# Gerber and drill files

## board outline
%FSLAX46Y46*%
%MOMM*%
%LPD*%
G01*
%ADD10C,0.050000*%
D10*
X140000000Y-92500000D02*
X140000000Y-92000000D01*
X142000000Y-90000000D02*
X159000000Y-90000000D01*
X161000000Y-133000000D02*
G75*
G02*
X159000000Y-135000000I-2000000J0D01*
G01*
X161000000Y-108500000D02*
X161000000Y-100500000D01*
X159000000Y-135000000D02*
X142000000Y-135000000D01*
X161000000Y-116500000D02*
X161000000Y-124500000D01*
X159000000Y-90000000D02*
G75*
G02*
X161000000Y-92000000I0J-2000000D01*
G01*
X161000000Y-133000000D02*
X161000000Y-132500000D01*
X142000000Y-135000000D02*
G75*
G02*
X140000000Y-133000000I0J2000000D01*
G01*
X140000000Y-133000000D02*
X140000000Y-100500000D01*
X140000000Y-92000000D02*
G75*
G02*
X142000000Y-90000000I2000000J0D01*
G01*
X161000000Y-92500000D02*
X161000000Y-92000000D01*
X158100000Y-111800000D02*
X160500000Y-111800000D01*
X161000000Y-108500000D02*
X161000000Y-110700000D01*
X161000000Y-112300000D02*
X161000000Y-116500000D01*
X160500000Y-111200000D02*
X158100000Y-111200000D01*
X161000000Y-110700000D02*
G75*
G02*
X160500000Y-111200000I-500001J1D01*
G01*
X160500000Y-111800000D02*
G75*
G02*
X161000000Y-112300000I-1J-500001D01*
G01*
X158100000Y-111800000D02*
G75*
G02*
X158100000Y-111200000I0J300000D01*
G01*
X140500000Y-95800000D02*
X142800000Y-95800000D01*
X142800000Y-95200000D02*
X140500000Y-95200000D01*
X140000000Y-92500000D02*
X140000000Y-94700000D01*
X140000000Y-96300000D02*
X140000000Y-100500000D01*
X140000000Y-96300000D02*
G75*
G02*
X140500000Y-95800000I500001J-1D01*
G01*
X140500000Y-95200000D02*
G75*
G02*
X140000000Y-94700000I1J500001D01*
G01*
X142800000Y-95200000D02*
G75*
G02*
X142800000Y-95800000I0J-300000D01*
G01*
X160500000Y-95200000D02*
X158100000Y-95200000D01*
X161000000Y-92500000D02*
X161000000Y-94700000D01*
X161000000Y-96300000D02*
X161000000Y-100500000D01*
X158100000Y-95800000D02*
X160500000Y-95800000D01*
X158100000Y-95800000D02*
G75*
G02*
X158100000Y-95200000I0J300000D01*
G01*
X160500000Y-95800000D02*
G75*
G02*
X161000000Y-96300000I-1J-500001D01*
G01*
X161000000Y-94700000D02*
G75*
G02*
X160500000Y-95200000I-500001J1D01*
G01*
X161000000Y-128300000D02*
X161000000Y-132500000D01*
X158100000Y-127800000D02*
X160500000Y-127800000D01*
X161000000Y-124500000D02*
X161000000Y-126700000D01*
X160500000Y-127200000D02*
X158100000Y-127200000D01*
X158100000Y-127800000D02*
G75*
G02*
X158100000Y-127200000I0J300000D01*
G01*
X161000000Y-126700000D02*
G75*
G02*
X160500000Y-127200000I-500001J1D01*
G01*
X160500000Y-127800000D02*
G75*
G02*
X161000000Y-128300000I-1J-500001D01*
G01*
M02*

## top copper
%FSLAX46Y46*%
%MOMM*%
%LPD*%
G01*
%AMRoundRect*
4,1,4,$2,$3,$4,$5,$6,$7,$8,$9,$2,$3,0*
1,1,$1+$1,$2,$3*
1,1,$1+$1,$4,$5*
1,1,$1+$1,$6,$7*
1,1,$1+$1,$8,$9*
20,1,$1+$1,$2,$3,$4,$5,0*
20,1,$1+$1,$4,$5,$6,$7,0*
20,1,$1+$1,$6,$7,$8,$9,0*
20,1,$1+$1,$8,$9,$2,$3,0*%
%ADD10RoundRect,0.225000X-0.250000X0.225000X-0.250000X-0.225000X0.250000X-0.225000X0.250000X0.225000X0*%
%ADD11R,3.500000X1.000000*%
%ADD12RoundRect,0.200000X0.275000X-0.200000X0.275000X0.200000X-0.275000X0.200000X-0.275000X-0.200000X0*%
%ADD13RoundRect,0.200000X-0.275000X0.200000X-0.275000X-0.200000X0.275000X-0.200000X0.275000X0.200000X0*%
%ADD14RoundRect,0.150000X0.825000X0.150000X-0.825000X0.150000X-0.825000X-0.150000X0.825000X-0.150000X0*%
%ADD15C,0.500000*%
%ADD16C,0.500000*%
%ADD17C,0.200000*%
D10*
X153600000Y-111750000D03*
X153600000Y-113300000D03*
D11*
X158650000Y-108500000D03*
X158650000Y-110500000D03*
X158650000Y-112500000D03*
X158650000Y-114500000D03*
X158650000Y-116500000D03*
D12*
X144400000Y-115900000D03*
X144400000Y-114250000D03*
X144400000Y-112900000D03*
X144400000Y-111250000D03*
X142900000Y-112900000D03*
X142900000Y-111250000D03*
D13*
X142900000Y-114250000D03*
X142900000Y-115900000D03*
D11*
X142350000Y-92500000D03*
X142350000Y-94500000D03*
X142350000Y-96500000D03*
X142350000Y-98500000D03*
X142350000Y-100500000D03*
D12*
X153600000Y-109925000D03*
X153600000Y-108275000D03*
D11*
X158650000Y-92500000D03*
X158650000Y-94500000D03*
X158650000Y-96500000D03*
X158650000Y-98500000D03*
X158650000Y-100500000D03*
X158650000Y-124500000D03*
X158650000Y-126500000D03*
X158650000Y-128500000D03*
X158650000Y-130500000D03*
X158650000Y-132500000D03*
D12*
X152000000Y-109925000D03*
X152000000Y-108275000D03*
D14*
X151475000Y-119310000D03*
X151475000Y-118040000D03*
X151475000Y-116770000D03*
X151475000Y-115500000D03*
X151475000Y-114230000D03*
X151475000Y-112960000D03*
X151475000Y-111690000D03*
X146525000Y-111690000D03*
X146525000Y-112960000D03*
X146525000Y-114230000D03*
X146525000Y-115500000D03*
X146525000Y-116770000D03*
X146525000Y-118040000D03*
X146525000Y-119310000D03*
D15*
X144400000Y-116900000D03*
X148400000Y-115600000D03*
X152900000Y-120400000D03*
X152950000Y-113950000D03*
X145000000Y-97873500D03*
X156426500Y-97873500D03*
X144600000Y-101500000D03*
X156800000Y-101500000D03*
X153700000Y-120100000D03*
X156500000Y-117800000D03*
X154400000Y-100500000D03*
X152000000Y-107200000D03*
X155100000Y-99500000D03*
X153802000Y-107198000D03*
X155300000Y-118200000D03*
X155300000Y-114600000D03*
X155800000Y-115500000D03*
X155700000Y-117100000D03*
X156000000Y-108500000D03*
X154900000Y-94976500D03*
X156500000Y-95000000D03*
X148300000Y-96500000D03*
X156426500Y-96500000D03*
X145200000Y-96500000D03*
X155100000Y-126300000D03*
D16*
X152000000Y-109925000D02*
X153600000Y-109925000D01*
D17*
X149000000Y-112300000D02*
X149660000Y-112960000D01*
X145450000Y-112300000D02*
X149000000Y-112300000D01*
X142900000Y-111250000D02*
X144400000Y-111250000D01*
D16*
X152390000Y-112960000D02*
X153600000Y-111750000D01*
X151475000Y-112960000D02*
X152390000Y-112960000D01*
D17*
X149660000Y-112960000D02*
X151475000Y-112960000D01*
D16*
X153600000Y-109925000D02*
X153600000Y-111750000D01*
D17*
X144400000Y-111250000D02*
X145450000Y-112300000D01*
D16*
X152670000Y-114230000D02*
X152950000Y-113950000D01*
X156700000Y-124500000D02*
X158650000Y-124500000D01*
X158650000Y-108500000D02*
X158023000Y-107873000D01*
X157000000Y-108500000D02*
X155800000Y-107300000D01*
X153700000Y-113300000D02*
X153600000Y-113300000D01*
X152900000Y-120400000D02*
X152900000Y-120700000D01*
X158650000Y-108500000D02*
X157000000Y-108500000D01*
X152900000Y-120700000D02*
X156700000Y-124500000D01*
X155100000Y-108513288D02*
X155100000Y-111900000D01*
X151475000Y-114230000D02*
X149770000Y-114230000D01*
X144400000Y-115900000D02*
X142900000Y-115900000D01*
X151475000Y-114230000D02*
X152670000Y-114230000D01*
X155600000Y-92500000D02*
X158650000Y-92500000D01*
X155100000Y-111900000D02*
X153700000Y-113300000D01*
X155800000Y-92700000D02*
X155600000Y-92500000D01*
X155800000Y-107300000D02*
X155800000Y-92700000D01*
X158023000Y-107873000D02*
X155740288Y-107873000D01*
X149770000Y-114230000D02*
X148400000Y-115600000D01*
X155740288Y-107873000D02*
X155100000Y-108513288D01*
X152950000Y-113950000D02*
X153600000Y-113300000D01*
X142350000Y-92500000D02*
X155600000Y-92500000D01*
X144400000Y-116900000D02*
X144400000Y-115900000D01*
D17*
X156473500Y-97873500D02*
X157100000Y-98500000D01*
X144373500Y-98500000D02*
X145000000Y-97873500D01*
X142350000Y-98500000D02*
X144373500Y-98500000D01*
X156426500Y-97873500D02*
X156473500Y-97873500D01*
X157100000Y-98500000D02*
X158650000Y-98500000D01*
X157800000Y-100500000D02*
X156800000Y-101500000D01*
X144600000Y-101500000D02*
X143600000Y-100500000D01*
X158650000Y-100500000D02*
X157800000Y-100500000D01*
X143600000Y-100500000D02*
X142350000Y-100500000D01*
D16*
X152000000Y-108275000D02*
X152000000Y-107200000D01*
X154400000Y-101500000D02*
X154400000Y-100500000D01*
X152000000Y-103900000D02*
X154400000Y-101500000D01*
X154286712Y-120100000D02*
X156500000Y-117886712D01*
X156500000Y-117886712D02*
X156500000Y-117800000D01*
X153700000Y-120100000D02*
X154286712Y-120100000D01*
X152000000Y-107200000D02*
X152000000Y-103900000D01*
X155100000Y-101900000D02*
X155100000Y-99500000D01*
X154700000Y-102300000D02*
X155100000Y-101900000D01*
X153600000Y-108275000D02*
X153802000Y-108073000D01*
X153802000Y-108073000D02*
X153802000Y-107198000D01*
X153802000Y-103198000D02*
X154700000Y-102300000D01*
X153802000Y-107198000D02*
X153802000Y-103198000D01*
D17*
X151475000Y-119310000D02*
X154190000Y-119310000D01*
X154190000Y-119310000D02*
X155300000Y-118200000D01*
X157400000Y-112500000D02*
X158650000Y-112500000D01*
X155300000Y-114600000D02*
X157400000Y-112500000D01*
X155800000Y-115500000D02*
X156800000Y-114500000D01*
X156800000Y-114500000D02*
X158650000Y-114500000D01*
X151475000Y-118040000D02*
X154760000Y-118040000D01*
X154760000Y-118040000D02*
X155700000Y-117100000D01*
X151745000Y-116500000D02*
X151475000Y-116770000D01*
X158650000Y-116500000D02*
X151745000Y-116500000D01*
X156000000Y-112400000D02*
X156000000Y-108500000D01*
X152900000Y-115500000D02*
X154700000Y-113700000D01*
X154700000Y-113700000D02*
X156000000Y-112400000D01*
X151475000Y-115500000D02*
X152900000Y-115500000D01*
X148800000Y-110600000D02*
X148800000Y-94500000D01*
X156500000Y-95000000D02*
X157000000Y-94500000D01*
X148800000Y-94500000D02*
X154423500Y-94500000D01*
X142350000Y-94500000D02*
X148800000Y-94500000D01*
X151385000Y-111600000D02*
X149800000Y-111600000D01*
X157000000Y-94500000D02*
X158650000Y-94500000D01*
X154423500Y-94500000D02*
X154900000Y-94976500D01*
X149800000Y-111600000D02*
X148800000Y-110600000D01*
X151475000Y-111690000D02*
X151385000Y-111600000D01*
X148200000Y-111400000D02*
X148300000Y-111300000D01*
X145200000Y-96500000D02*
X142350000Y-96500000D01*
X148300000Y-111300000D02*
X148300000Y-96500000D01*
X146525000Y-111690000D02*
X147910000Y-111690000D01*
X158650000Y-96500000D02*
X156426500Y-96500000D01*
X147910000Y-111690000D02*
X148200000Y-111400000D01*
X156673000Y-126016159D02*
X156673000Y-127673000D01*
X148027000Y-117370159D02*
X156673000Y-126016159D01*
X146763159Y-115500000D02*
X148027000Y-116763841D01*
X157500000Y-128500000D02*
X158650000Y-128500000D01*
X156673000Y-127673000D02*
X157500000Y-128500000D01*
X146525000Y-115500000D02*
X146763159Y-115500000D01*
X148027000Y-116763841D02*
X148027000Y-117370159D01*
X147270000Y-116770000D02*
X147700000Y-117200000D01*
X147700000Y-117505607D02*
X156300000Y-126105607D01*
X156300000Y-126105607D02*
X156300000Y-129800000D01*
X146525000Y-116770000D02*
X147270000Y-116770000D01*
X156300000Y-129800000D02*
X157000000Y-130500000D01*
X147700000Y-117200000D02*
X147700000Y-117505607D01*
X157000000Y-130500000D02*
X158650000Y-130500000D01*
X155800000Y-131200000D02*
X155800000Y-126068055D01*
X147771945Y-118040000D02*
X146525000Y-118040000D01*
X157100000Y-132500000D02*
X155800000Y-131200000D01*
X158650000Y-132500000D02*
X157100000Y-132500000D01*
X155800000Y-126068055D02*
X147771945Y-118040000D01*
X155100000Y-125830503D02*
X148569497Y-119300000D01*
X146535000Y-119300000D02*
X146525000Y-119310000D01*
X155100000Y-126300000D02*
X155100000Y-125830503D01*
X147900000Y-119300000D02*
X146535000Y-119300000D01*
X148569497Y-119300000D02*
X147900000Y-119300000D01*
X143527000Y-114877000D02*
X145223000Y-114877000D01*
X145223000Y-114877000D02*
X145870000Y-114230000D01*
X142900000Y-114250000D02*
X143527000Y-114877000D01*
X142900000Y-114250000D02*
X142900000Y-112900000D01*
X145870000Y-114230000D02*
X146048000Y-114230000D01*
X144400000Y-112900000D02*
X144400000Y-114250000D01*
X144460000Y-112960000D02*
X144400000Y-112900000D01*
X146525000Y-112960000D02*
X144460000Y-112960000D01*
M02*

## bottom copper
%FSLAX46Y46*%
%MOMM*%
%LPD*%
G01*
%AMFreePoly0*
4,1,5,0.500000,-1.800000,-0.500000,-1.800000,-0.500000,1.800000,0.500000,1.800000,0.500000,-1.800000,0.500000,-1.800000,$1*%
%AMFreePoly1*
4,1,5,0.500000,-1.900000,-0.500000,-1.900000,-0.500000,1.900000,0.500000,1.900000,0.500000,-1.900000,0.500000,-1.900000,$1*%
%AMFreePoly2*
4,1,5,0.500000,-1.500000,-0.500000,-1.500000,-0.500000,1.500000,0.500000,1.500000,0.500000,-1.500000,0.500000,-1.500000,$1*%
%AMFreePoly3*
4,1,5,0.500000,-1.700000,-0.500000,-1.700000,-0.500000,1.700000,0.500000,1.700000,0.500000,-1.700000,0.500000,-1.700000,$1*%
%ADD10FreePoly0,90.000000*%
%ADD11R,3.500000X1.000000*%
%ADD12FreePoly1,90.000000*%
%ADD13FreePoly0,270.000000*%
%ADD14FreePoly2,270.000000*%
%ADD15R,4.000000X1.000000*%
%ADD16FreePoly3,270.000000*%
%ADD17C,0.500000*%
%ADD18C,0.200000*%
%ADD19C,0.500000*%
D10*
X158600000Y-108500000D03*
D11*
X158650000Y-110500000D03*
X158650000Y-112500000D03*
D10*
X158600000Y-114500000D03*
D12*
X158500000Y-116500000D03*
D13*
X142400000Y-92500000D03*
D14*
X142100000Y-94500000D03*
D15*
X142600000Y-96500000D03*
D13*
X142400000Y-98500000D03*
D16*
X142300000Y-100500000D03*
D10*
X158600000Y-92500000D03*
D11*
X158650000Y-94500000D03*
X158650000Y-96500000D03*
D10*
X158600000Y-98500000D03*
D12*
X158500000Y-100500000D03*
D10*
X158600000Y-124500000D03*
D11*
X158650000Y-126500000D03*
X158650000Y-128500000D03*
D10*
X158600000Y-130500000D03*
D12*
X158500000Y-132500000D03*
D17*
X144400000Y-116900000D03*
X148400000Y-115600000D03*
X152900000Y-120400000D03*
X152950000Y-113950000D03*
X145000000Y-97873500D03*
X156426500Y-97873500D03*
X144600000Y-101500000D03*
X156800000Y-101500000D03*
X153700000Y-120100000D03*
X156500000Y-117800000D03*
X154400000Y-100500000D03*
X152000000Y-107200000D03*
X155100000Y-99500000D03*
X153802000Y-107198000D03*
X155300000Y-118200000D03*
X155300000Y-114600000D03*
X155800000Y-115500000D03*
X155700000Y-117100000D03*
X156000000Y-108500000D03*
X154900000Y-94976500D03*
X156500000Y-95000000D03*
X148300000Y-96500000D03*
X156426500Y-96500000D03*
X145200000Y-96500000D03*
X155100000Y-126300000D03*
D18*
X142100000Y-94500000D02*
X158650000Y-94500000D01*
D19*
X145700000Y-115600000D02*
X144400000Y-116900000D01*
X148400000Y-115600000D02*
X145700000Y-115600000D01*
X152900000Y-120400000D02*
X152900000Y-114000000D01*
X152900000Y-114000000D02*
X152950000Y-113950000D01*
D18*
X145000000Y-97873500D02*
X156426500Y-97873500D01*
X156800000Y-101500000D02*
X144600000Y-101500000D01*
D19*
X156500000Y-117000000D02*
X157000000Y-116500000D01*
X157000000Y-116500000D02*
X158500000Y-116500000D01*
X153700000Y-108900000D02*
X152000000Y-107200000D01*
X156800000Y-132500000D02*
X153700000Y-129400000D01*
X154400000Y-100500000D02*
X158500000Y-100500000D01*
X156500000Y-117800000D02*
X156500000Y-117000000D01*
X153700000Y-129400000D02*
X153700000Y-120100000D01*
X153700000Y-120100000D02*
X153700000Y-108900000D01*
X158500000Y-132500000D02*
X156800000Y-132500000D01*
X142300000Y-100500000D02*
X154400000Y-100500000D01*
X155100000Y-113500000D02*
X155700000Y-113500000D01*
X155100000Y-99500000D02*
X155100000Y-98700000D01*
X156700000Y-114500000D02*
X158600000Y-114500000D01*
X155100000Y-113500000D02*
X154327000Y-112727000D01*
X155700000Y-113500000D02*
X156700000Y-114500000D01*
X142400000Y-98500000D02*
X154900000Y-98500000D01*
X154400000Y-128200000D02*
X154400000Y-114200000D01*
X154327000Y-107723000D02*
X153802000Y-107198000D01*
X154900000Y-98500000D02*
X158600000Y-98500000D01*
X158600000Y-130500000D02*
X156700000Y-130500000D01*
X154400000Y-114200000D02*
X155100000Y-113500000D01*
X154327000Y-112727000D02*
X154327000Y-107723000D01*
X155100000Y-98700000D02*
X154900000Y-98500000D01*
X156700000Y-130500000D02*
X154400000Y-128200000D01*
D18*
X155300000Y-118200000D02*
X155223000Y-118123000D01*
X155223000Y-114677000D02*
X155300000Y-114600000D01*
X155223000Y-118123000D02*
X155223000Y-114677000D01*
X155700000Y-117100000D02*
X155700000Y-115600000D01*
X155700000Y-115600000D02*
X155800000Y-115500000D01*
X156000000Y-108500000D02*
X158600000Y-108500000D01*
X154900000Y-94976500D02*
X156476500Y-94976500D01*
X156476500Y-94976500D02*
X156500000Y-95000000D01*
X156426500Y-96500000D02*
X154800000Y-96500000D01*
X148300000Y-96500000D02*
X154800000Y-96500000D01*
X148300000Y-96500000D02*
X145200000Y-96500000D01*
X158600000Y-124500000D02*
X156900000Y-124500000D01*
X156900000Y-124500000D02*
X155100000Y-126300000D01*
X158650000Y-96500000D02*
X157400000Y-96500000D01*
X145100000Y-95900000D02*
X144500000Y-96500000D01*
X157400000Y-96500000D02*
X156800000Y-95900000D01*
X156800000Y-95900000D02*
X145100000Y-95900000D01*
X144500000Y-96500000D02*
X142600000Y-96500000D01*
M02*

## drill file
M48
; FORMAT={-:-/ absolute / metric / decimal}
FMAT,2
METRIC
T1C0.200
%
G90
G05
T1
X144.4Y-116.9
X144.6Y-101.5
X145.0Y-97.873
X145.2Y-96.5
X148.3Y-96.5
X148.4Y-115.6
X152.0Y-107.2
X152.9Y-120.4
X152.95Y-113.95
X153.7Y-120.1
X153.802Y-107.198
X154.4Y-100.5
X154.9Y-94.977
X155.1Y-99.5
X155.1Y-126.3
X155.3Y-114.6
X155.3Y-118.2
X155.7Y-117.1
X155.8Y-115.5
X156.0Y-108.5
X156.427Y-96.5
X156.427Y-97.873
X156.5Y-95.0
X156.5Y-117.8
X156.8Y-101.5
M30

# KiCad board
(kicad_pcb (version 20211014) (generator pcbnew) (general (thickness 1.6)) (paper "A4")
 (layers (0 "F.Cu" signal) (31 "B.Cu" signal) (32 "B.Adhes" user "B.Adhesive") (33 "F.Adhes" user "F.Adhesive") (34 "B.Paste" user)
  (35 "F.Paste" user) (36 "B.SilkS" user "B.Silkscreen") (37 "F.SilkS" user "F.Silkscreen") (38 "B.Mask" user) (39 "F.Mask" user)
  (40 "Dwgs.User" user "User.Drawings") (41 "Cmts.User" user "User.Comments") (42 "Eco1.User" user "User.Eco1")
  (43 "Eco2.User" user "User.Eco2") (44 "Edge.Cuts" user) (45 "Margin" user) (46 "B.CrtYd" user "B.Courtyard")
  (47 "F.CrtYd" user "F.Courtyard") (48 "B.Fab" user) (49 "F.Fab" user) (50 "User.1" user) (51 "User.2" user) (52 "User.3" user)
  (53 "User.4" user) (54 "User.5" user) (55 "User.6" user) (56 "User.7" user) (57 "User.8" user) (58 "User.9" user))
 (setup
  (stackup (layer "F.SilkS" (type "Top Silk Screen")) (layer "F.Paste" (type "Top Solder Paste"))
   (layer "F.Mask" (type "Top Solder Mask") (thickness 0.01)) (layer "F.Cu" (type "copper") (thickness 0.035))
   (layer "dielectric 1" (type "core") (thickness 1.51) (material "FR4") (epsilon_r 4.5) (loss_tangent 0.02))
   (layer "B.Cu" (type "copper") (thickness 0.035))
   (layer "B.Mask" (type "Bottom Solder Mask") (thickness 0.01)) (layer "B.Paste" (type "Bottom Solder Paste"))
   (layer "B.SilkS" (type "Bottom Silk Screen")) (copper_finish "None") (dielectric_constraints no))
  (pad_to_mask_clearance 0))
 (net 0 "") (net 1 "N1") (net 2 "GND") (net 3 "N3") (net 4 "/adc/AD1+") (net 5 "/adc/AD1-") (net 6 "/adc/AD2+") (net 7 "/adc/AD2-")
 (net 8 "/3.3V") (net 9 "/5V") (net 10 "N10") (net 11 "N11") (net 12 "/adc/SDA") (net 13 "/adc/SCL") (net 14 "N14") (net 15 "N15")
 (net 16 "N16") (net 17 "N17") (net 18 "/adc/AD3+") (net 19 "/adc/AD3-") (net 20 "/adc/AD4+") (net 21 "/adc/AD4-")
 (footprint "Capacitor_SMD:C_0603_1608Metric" (layer "F.Cu") (at 153.6 112.525 -90)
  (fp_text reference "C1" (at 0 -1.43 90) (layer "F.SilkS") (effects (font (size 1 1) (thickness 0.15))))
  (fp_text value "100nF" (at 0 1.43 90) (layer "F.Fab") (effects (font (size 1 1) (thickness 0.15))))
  (pad "1" smd roundrect (at -0.775 0 270) (size 0.9 0.95) (layers "F.Cu" "F.Paste" "F.Mask") (roundrect_rratio 0.25) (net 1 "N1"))
  (pad "2" smd roundrect (at 0.775 0 270) (size 0.9 0.95) (layers "F.Cu" "F.Paste" "F.Mask") (roundrect_rratio 0.25) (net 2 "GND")))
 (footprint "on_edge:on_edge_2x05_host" (layer "F.Cu") (at 161 112.5 -90)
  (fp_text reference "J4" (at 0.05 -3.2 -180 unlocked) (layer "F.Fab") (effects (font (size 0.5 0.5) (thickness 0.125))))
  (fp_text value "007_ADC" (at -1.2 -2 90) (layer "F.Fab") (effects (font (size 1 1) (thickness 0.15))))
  (fp_line (start -0.7 2.9) (end -0.7 0.5) (layer "Edge.Cuts") (width 0.05))
  (fp_line (start -4 0) (end -1.8 0) (layer "Edge.Cuts") (width 0.05))
  (fp_line (start -0.2 0) (end 4 0) (layer "Edge.Cuts") (width 0.05))
  (fp_line (start -1.3 0.5) (end -1.3 2.9) (layer "Edge.Cuts") (width 0.05))
  (fp_arc (start -1.8 0) (mid -1.446447 0.146447) (end -1.3 0.5) (layer "Edge.Cuts") (width 0.05))
  (fp_arc (start -0.7 0.5) (mid -0.553553 0.146447) (end -0.2 0) (layer "Edge.Cuts") (width 0.05))
  (fp_arc (start -0.7 2.9) (mid -1 3.2) (end -1.3 2.9) (layer "Edge.Cuts") (width 0.05))
  (pad "1" smd rect (at -4 2.35 270) (size 1 3.5) (layers "F.Cu" "F.Mask") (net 2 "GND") (zone_connect 0))
  (pad "2" smd rect (at -2 2.35 270) (size 1 3.5) (layers "F.Cu" "F.Mask") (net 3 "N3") (zone_connect 0))
  (pad "3" smd rect (at 0 2.35 270) (size 1 3.5) (layers "F.Cu" "F.Mask") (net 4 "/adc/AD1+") (zone_connect 0))
  (pad "4" smd rect (at 2 2.35 270) (size 1 3.5) (layers "F.Cu" "F.Mask") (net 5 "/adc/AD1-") (zone_connect 0))
  (pad "5" smd rect (at 4 2.35 270) (size 1 3.5) (layers "F.Cu" "F.Mask") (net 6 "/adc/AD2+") (zone_connect 0))
  (pad "6" smd custom (at -4 2.4 90) (size 1 3.6) (layers "B.Cu" "B.Mask") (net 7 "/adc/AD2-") (zone_connect 0)
   (options (clearance outline) (anchor rect)) (primitives))
  (pad "7" smd rect (at -2 2.35 90) (size 1 3.5) (layers "B.Cu" "B.Mask") (zone_connect 0))
  (pad "8" smd rect (at 0 2.35 90) (size 1 3.5) (layers "B.Cu" "B.Mask") (zone_connect 0))
  (pad "9" smd custom (at 2 2.4 90) (size 1 3.6) (layers "B.Cu" "B.Mask") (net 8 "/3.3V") (zone_connect 0)
   (options (clearance outline) (anchor rect)) (primitives))
  (pad "10" smd custom (at 4 2.5 90) (size 1 3.8) (layers "B.Cu" "B.Mask") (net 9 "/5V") (zone_connect 0)
   (options (clearance outline) (anchor rect)) (primitives)))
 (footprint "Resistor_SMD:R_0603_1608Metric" (layer "F.Cu") (at 144.4 115.075 90)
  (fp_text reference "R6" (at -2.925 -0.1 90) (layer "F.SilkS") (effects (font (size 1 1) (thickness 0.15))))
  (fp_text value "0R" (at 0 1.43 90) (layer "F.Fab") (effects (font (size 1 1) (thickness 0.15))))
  (pad "1" smd roundrect (at -0.825 0 90) (size 0.8 0.95) (layers "F.Cu" "F.Paste" "F.Mask") (roundrect_rratio 0.25) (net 2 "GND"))
  (pad "2" smd roundrect (at 0.825 0 90) (size 0.8 0.95) (layers "F.Cu" "F.Paste" "F.Mask") (roundrect_rratio 0.25) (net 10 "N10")))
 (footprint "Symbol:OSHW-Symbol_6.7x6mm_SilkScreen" (layer "F.Cu") (at 150 131)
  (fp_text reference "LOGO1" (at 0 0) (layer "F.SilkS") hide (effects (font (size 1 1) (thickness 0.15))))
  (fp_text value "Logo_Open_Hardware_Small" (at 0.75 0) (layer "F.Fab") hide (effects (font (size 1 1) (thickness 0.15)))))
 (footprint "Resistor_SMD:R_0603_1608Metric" (layer "F.Cu") (at 144.4 112.075 90)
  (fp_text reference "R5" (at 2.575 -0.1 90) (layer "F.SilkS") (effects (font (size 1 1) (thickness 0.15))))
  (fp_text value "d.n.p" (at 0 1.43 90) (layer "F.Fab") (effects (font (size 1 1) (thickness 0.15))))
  (pad "1" smd roundrect (at -0.825 0 90) (size 0.8 0.95) (layers "F.Cu" "F.Paste" "F.Mask") (roundrect_rratio 0.25) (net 10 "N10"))
  (pad "2" smd roundrect (at 0.825 0 90) (size 0.8 0.95) (layers "F.Cu" "F.Paste" "F.Mask") (roundrect_rratio 0.25) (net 1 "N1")))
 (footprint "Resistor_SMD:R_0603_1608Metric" (layer "F.Cu") (at 142.9 112.075 90)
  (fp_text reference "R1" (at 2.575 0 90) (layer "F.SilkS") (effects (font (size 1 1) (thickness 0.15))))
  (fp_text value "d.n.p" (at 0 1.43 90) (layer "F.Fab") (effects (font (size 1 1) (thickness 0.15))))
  (pad "1" smd roundrect (at -0.825 0 90) (size 0.8 0.95) (layers "F.Cu" "F.Paste" "F.Mask") (roundrect_rratio 0.25) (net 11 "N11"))
  (pad "2" smd roundrect (at 0.825 0 90) (size 0.8 0.95) (layers "F.Cu" "F.Paste" "F.Mask") (roundrect_rratio 0.25) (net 1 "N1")))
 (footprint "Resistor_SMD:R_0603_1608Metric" (layer "F.Cu") (at 142.9 115.075 -90)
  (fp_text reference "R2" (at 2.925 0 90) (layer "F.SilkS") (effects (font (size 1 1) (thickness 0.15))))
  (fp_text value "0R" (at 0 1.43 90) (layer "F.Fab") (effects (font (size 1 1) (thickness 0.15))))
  (pad "1" smd roundrect (at -0.825 0 270) (size 0.8 0.95) (layers "F.Cu" "F.Paste" "F.Mask") (roundrect_rratio 0.25) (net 11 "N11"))
  (pad "2" smd roundrect (at 0.825 0 270) (size 0.8 0.95) (layers "F.Cu" "F.Paste" "F.Mask") (roundrect_rratio 0.25) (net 2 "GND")))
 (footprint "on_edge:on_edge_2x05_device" (layer "F.Cu") (at 140 96.5 -90)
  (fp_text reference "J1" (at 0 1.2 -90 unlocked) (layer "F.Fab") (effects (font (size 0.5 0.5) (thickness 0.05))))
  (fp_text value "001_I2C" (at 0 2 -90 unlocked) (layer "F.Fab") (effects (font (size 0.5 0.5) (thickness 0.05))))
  (fp_line (start -0.7 -0.5) (end -0.7 -2.8) (layer "Edge.Cuts") (width 0.05))
  (fp_line (start -1.3 -2.8) (end -1.3 -0.5) (layer "Edge.Cuts") (width 0.05))
  (fp_line (start -4 0) (end -1.8 0) (layer "Edge.Cuts") (width 0.05))
  (fp_line (start -0.2 0) (end 4 0) (layer "Edge.Cuts") (width 0.05))
  (fp_arc (start -0.2 0) (mid -0.553553 -0.146447) (end -0.7 -0.5) (layer "Edge.Cuts") (width 0.05))
  (fp_arc (start -1.3 -0.5) (mid -1.446447 -0.146447) (end -1.8 0) (layer "Edge.Cuts") (width 0.05))
  (fp_arc (start -1.3 -2.8) (mid -1 -3.1) (end -0.7 -2.8) (layer "Edge.Cuts") (width 0.05))
  (pad "1" smd rect (at -4 -2.35 90) (size 1 3.5) (layers "F.Cu" "F.Mask") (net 2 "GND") (zone_connect 0))
  (pad "2" smd rect (at -2 -2.35 270) (size 1 3.5) (layers "F.Cu" "F.Mask") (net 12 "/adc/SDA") (zone_connect 0))
  (pad "3" smd rect (at 0 -2.35 270) (size 1 3.5) (layers "F.Cu" "F.Mask") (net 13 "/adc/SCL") (zone_connect 0))
  (pad "4" smd rect (at 2 -2.35 90) (size 1 3.5) (layers "F.Cu" "F.Mask") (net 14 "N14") (zone_connect 0))
  (pad "5" smd rect (at 4 -2.35 90) (size 1 3.5) (layers "F.Cu" "F.Mask") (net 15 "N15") (zone_connect 0))
  (pad "6" smd custom (at -4 -2.4 270) (size 1 3.6) (layers "B.Cu" "B.Mask") (zone_connect 0) (options (clearance outline) (anchor rect))
   (primitives))
  (pad "7" smd custom (at -2 -2.1 270) (size 1 3) (layers "B.Cu" "B.Mask") (zone_connect 0) (options (clearance outline) (anchor rect))
   (primitives))
  (pad "8" smd rect (at 0 -2.6 270) (size 1 4) (layers "B.Cu" "B.Mask") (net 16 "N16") (zone_connect 0))
  (pad "9" smd custom (at 2 -2.4 270) (size 1 3.6) (layers "B.Cu" "B.Mask") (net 8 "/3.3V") (zone_connect 0)
   (options (clearance outline) (anchor rect)) (primitives))
  (pad "10" smd custom (at 4 -2.3 270) (size 1 3.4) (layers "B.Cu" "B.Mask") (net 9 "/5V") (zone_connect 0)
   (options (clearance outline) (anchor rect)) (primitives)))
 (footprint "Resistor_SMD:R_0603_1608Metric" (layer "F.Cu") (at 153.6 109.1 90)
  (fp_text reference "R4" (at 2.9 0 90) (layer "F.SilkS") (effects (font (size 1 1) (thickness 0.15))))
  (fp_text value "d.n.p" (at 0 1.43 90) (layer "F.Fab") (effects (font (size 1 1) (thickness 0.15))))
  (pad "1" smd roundrect (at -0.825 0 90) (size 0.8 0.95) (layers "F.Cu" "F.Paste" "F.Mask") (roundrect_rratio 0.25) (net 1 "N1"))
  (pad "2" smd roundrect (at 0.825 0 90) (size 0.8 0.95) (layers "F.Cu" "F.Paste" "F.Mask") (roundrect_rratio 0.25) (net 8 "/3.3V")))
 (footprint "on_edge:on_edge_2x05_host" (layer "F.Cu") (at 161 96.5 -90)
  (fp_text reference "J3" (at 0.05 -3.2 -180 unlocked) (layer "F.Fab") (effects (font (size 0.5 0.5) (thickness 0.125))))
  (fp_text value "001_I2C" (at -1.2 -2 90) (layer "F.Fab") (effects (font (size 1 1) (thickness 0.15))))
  (fp_line (start -1.3 0.5) (end -1.3 2.9) (layer "Edge.Cuts") (width 0.05))
  (fp_line (start -4 0) (end -1.8 0) (layer "Edge.Cuts") (width 0.05))
  (fp_line (start -0.2 0) (end 4 0) (layer "Edge.Cuts") (width 0.05))
  (fp_line (start -0.7 2.9) (end -0.7 0.5) (layer "Edge.Cuts") (width 0.05))
  (fp_arc (start -0.7 2.9) (mid -1 3.2) (end -1.3 2.9) (layer "Edge.Cuts") (width 0.05))
  (fp_arc (start -0.7 0.5) (mid -0.553553 0.146447) (end -0.2 0) (layer "Edge.Cuts") (width 0.05))
  (fp_arc (start -1.8 0) (mid -1.446447 0.146447) (end -1.3 0.5) (layer "Edge.Cuts") (width 0.05))
  (pad "1" smd rect (at -4 2.35 270) (size 1 3.5) (layers "F.Cu" "F.Mask") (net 2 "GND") (zone_connect 0))
  (pad "2" smd rect (at -2 2.35 270) (size 1 3.5) (layers "F.Cu" "F.Mask") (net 12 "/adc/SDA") (zone_connect 0))
  (pad "3" smd rect (at 0 2.35 270) (size 1 3.5) (layers "F.Cu" "F.Mask") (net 13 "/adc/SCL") (zone_connect 0))
  (pad "4" smd rect (at 2 2.35 270) (size 1 3.5) (layers "F.Cu" "F.Mask") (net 14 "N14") (zone_connect 0))
  (pad "5" smd rect (at 4 2.35 270) (size 1 3.5) (layers "F.Cu" "F.Mask") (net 15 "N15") (zone_connect 0))
  (pad "6" smd custom (at -4 2.4 90) (size 1 3.6) (layers "B.Cu" "B.Mask") (zone_connect 0) (options (clearance outline) (anchor rect))
   (primitives))
  (pad "7" smd rect (at -2 2.35 90) (size 1 3.5) (layers "B.Cu" "B.Mask") (zone_connect 0))
  (pad "8" smd rect (at 0 2.35 90) (size 1 3.5) (layers "B.Cu" "B.Mask") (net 16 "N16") (zone_connect 0))
  (pad "9" smd custom (at 2 2.4 90) (size 1 3.6) (layers "B.Cu" "B.Mask") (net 8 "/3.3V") (zone_connect 0)
   (options (clearance outline) (anchor rect)) (primitives))
  (pad "10" smd custom (at 4 2.5 90) (size 1 3.8) (layers "B.Cu" "B.Mask") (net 9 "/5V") (zone_connect 0)
   (options (clearance outline) (anchor rect)) (primitives)))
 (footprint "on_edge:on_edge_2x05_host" (layer "F.Cu") (at 161 128.5 -90)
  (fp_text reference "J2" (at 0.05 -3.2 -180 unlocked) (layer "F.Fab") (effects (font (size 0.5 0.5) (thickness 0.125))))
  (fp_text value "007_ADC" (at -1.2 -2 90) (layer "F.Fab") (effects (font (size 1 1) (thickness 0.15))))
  (fp_line (start -0.2 0) (end 4 0) (layer "Edge.Cuts") (width 0.05))
  (fp_line (start -0.7 2.9) (end -0.7 0.5) (layer "Edge.Cuts") (width 0.05))
  (fp_line (start -4 0) (end -1.8 0) (layer "Edge.Cuts") (width 0.05))
  (fp_line (start -1.3 0.5) (end -1.3 2.9) (layer "Edge.Cuts") (width 0.05))
  (fp_arc (start -0.7 2.9) (mid -1 3.2) (end -1.3 2.9) (layer "Edge.Cuts") (width 0.05))
  (fp_arc (start -1.8 0) (mid -1.446447 0.146447) (end -1.3 0.5) (layer "Edge.Cuts") (width 0.05))
  (fp_arc (start -0.7 0.5) (mid -0.553553 0.146447) (end -0.2 0) (layer "Edge.Cuts") (width 0.05))
  (pad "1" smd rect (at -4 2.35 270) (size 1 3.5) (layers "F.Cu" "F.Mask") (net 2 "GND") (zone_connect 0))
  (pad "2" smd rect (at -2 2.35 270) (size 1 3.5) (layers "F.Cu" "F.Mask") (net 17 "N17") (zone_connect 0))
  (pad "3" smd rect (at 0 2.35 270) (size 1 3.5) (layers "F.Cu" "F.Mask") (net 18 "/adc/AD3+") (zone_connect 0))
  (pad "4" smd rect (at 2 2.35 270) (size 1 3.5) (layers "F.Cu" "F.Mask") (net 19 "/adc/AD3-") (zone_connect 0))
  (pad "5" smd rect (at 4 2.35 270) (size 1 3.5) (layers "F.Cu" "F.Mask") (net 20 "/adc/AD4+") (zone_connect 0))
  (pad "6" smd custom (at -4 2.4 90) (size 1 3.6) (layers "B.Cu" "B.Mask") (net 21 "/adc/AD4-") (zone_connect 0)
   (options (clearance outline) (anchor rect)) (primitives))
  (pad "7" smd rect (at -2 2.35 90) (size 1 3.5) (layers "B.Cu" "B.Mask") (zone_connect 0))
  (pad "8" smd rect (at 0 2.35 90) (size 1 3.5) (layers "B.Cu" "B.Mask") (zone_connect 0))
  (pad "9" smd custom (at 2 2.4 90) (size 1 3.6) (layers "B.Cu" "B.Mask") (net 8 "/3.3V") (zone_connect 0)
   (options (clearance outline) (anchor rect)) (primitives))
  (pad "10" smd custom (at 4 2.5 90) (size 1 3.8) (layers "B.Cu" "B.Mask") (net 9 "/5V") (zone_connect 0)
   (options (clearance outline) (anchor rect)) (primitives)))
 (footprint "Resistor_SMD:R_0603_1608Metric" (layer "F.Cu") (at 152 109.1 90)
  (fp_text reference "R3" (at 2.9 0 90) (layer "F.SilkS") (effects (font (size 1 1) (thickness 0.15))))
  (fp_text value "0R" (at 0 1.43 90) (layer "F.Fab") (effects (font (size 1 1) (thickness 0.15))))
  (pad "1" smd roundrect (at -0.825 0 90) (size 0.8 0.95) (layers "F.Cu" "F.Paste" "F.Mask") (roundrect_rratio 0.25) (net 1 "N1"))
  (pad "2" smd roundrect (at 0.825 0 90) (size 0.8 0.95) (layers "F.Cu" "F.Paste" "F.Mask") (roundrect_rratio 0.25) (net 9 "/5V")))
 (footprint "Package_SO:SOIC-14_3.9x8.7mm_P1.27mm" (layer "F.Cu") (at 149 115.5 180)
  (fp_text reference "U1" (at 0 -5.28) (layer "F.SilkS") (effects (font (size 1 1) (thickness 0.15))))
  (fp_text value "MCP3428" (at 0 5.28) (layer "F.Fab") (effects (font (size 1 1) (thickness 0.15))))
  (pad "1" smd roundrect (at -2.475 -3.81 180) (size 1.95 0.6) (layers "F.Cu" "F.Paste" "F.Mask") (roundrect_rratio 0.25)
   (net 4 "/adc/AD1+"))
  (pad "2" smd roundrect (at -2.475 -2.54 180) (size 1.95 0.6) (layers "F.Cu" "F.Paste" "F.Mask") (roundrect_rratio 0.25)
   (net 5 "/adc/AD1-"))
  (pad "3" smd roundrect (at -2.475 -1.27 180) (size 1.95 0.6) (layers "F.Cu" "F.Paste" "F.Mask") (roundrect_rratio 0.25)
   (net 6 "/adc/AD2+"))
  (pad "4" smd roundrect (at -2.475 0 180) (size 1.95 0.6) (layers "F.Cu" "F.Paste" "F.Mask") (roundrect_rratio 0.25) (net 7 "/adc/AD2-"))
  (pad "5" smd roundrect (at -2.475 1.27 180) (size 1.95 0.6) (layers "F.Cu" "F.Paste" "F.Mask") (roundrect_rratio 0.25) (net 2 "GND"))
  (pad "6" smd roundrect (at -2.475 2.54 180) (size 1.95 0.6) (layers "F.Cu" "F.Paste" "F.Mask") (roundrect_rratio 0.25) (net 1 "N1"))
  (pad "7" smd roundrect (at -2.475 3.81 180) (size 1.95 0.6) (layers "F.Cu" "F.Paste" "F.Mask") (roundrect_rratio 0.25) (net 12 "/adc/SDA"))
  (pad "8" smd roundrect (at 2.475 3.81 180) (size 1.95 0.6) (layers "F.Cu" "F.Paste" "F.Mask") (roundrect_rratio 0.25) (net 13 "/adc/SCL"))
  (pad "9" smd roundrect (at 2.475 2.54 180) (size 1.95 0.6) (layers "F.Cu" "F.Paste" "F.Mask") (roundrect_rratio 0.25) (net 10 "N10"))
  (pad "10" smd roundrect (at 2.475 1.27 180) (size 1.95 0.6) (layers "F.Cu" "F.Paste" "F.Mask") (roundrect_rratio 0.25) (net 11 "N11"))
  (pad "11" smd roundrect (at 2.475 0 180) (size 1.95 0.6) (layers "F.Cu" "F.Paste" "F.Mask") (roundrect_rratio 0.25) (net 18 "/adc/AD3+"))
  (pad "12" smd roundrect (at 2.475 -1.27 180) (size 1.95 0.6) (layers "F.Cu" "F.Paste" "F.Mask") (roundrect_rratio 0.25)
   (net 19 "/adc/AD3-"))
  (pad "13" smd roundrect (at 2.475 -2.54 180) (size 1.95 0.6) (layers "F.Cu" "F.Paste" "F.Mask") (roundrect_rratio 0.25)
   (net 20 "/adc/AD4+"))
  (pad "14" smd roundrect (at 2.475 -3.81 180) (size 1.95 0.6) (layers "F.Cu" "F.Paste" "F.Mask") (roundrect_rratio 0.25)
   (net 21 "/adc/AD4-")))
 (gr_line (start 140 92.5) (end 140 92) (layer "Edge.Cuts") (width 0.05))
 (gr_line (start 142 90) (end 159 90) (layer "Edge.Cuts") (width 0.05))
 (gr_arc (start 161 133) (mid 160.414214 134.414214) (end 159 135) (layer "Edge.Cuts") (width 0.05))
 (gr_line (start 161 108.5) (end 161 100.5) (layer "Edge.Cuts") (width 0.05))
 (gr_line (start 159 135) (end 142 135) (layer "Edge.Cuts") (width 0.05))
 (gr_line (start 161 116.5) (end 161 124.5) (layer "Edge.Cuts") (width 0.05))
 (gr_arc (start 159 90) (mid 160.414214 90.585786) (end 161 92) (layer "Edge.Cuts") (width 0.05))
 (gr_line (start 161 133) (end 161 132.5) (layer "Edge.Cuts") (width 0.05))
 (gr_arc (start 142 135) (mid 140.585786 134.414214) (end 140 133) (layer "Edge.Cuts") (width 0.05))
 (gr_line (start 140 133) (end 140 100.5) (layer "Edge.Cuts") (width 0.05))
 (gr_arc (start 140 92) (mid 140.585786 90.585786) (end 142 90) (layer "Edge.Cuts") (width 0.05))
 (gr_line (start 161 92.5) (end 161 92) (layer "Edge.Cuts") (width 0.05))
 (segment (start 142.1 94.5) (end 158.65 94.5) (width 0.2) (layer "B.Cu") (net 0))
 (segment (start 152 109.925) (end 153.6 109.925) (width 0.5) (layer "F.Cu") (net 1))
 (segment (start 149 112.3) (end 149.66 112.96) (width 0.2) (layer "F.Cu") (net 1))
 (segment (start 145.45 112.3) (end 149 112.3) (width 0.2) (layer "F.Cu") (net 1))
 (segment (start 142.9 111.25) (end 144.4 111.25) (width 0.2) (layer "F.Cu") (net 1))
 (segment (start 152.39 112.96) (end 153.6 111.75) (width 0.5) (layer "F.Cu") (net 1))
 (segment (start 151.475 112.96) (end 152.39 112.96) (width 0.5) (layer "F.Cu") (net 1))
 (segment (start 149.66 112.96) (end 151.475 112.96) (width 0.2) (layer "F.Cu") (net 1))
 (segment (start 153.6 109.925) (end 153.6 111.75) (width 0.5) (layer "F.Cu") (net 1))
 (segment (start 144.4 111.25) (end 145.45 112.3) (width 0.2) (layer "F.Cu") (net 1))
 (segment (start 152.67 114.23) (end 152.95 113.95) (width 0.5) (layer "F.Cu") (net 2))
 (segment (start 156.7 124.5) (end 158.65 124.5) (width 0.5) (layer "F.Cu") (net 2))
 (segment (start 158.65 108.5) (end 158.023 107.873) (width 0.5) (layer "F.Cu") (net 2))
 (segment (start 157 108.5) (end 155.8 107.3) (width 0.5) (layer "F.Cu") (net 2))
 (segment (start 153.7 113.3) (end 153.6 113.3) (width 0.5) (layer "F.Cu") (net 2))
 (segment (start 152.9 120.4) (end 152.9 120.7) (width 0.5) (layer "F.Cu") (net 2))
 (segment (start 158.65 108.5) (end 157 108.5) (width 0.5) (layer "F.Cu") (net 2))
 (segment (start 152.9 120.7) (end 156.7 124.5) (width 0.5) (layer "F.Cu") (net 2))
 (segment (start 155.1 108.513288) (end 155.1 111.9) (width 0.5) (layer "F.Cu") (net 2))
 (segment (start 151.475 114.23) (end 149.77 114.23) (width 0.5) (layer "F.Cu") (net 2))
 (segment (start 144.4 115.9) (end 142.9 115.9) (width 0.5) (layer "F.Cu") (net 2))
 (segment (start 151.475 114.23) (end 152.67 114.23) (width 0.5) (layer "F.Cu") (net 2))
 (segment (start 155.6 92.5) (end 158.65 92.5) (width 0.5) (layer "F.Cu") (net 2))
 (segment (start 155.1 111.9) (end 153.7 113.3) (width 0.5) (layer "F.Cu") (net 2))
 (segment (start 155.8 92.7) (end 155.6 92.5) (width 0.5) (layer "F.Cu") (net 2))
 (segment (start 155.8 107.3) (end 155.8 92.7) (width 0.5) (layer "F.Cu") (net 2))
 (segment (start 158.023 107.873) (end 155.740288 107.873) (width 0.5) (layer "F.Cu") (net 2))
 (segment (start 149.77 114.23) (end 148.4 115.6) (width 0.5) (layer "F.Cu") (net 2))
 (segment (start 155.740288 107.873) (end 155.1 108.513288) (width 0.5) (layer "F.Cu") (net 2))
 (segment (start 152.95 113.95) (end 153.6 113.3) (width 0.5) (layer "F.Cu") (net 2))
 (segment (start 142.35 92.5) (end 155.6 92.5) (width 0.5) (layer "F.Cu") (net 2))
 (segment (start 144.4 116.9) (end 144.4 115.9) (width 0.5) (layer "F.Cu") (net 2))
 (via (at 144.4 116.9) (size 0.5) (drill 0.2) (layers "F.Cu" "B.Cu") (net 2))
 (via (at 148.4 115.6) (size 0.5) (drill 0.2) (layers "F.Cu" "B.Cu") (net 2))
 (via (at 152.9 120.4) (size 0.5) (drill 0.2) (layers "F.Cu" "B.Cu") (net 2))
 (via (at 152.95 113.95) (size 0.5) (drill 0.2) (layers "F.Cu" "B.Cu") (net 2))
 (segment (start 145.7 115.6) (end 144.4 116.9) (width 0.5) (layer "B.Cu") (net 2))
 (segment (start 148.4 115.6) (end 145.7 115.6) (width 0.5) (layer "B.Cu") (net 2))
 (segment (start 152.9 120.4) (end 152.9 114) (width 0.5) (layer "B.Cu") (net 2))
 (segment (start 152.9 114) (end 152.95 113.95) (width 0.5) (layer "B.Cu") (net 2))
 (segment (start 156.4735 97.8735) (end 157.1 98.5) (width 0.2) (layer "F.Cu") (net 14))
 (segment (start 144.3735 98.5) (end 145 97.8735) (width 0.2) (layer "F.Cu") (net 14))
 (segment (start 142.35 98.5) (end 144.3735 98.5) (width 0.2) (layer "F.Cu") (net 14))
 (segment (start 156.4265 97.8735) (end 156.4735 97.8735) (width 0.2) (layer "F.Cu") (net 14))
 (segment (start 157.1 98.5) (end 158.65 98.5) (width 0.2) (layer "F.Cu") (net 14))
 (via (at 145 97.8735) (size 0.5) (drill 0.2) (layers "F.Cu" "B.Cu") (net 14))
 (via (at 156.4265 97.8735) (size 0.5) (drill 0.2) (layers "F.Cu" "B.Cu") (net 14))
 (segment (start 145 97.8735) (end 156.4265 97.8735) (width 0.2) (layer "B.Cu") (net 14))
 (segment (start 157.8 100.5) (end 156.8 101.5) (width 0.2) (layer "F.Cu") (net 15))
 (segment (start 144.6 101.5) (end 143.6 100.5) (width 0.2) (layer "F.Cu") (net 15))
 (segment (start 158.65 100.5) (end 157.8 100.5) (width 0.2) (layer "F.Cu") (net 15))
 (segment (start 143.6 100.5) (end 142.35 100.5) (width 0.2) (layer "F.Cu") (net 15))
 (via (at 144.6 101.5) (size 0.5) (drill 0.2) (layers "F.Cu" "B.Cu") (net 15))
 (via (at 156.8 101.5) (size 0.5) (drill 0.2) (layers "F.Cu" "B.Cu") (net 15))
 (segment (start 156.8 101.5) (end 144.6 101.5) (width 0.2) (layer "B.Cu") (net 15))
 (segment (start 152 108.275) (end 152 107.2) (width 0.5) (layer "F.Cu") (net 9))
 (segment (start 154.4 101.5) (end 154.4 100.5) (width 0.5) (layer "F.Cu") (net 9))
 (segment (start 152 103.9) (end 154.4 101.5) (width 0.5) (layer "F.Cu") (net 9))
 (segment (start 154.286712 120.1) (end 156.5 117.886712) (width 0.5) (layer "F.Cu") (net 9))
 (segment (start 156.5 117.886712) (end 156.5 117.8) (width 0.5) (layer "F.Cu") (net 9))
 (segment (start 153.7 120.1) (end 154.286712 120.1) (width 0.5) (layer "F.Cu") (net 9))
 (segment (start 152 107.2) (end 152 103.9) (width 0.5) (layer "F.Cu") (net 9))
 (via (at 153.7 120.1) (size 0.5) (drill 0.2) (layers "F.Cu" "B.Cu") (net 9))
 (via (at 156.5 117.8) (size 0.5) (drill 0.2) (layers "F.Cu" "B.Cu") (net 9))
 (via (at 154.4 100.5) (size 0.5) (drill 0.2) (layers "F.Cu" "B.Cu") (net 9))
 (via (at 152 107.2) (size 0.5) (drill 0.2) (layers "F.Cu" "B.Cu") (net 9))
 (segment (start 156.5 117) (end 157 116.5) (width 0.5) (layer "B.Cu") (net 9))
 (segment (start 157 116.5) (end 158.5 116.5) (width 0.5) (layer "B.Cu") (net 9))
 (segment (start 153.7 108.9) (end 152 107.2) (width 0.5) (layer "B.Cu") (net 9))
 (segment (start 156.8 132.5) (end 153.7 129.4) (width 0.5) (layer "B.Cu") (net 9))
 (segment (start 154.4 100.5) (end 158.5 100.5) (width 0.5) (layer "B.Cu") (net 9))
 (segment (start 156.5 117.8) (end 156.5 117) (width 0.5) (layer "B.Cu") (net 9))
 (segment (start 153.7 129.4) (end 153.7 120.1) (width 0.5) (layer "B.Cu") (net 9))
 (segment (start 153.7 120.1) (end 153.7 108.9) (width 0.5) (layer "B.Cu") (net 9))
 (segment (start 158.5 132.5) (end 156.8 132.5) (width 0.5) (layer "B.Cu") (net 9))
 (segment (start 142.3 100.5) (end 154.4 100.5) (width 0.5) (layer "B.Cu") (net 9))
 (segment (start 155.1 101.9) (end 155.1 99.5) (width 0.5) (layer "F.Cu") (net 8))
 (segment (start 154.7 102.3) (end 155.1 101.9) (width 0.5) (layer "F.Cu") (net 8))
 (segment (start 153.6 108.275) (end 153.802 108.073) (width 0.5) (layer "F.Cu") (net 8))
 (segment (start 153.802 108.073) (end 153.802 107.198) (width 0.5) (layer "F.Cu") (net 8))
 (segment (start 153.802 103.198) (end 154.7 102.3) (width 0.5) (layer "F.Cu") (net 8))
 (segment (start 153.802 107.198) (end 153.802 103.198) (width 0.5) (layer "F.Cu") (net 8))
 (via (at 155.1 99.5) (size 0.5) (drill 0.2) (layers "F.Cu" "B.Cu") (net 8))
 (via (at 153.802 107.198) (size 0.5) (drill 0.2) (layers "F.Cu" "B.Cu") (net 8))
 (segment (start 155.1 113.5) (end 155.7 113.5) (width 0.5) (layer "B.Cu") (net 8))
 (segment (start 155.1 99.5) (end 155.1 98.7) (width 0.5) (layer "B.Cu") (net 8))
 (segment (start 156.7 114.5) (end 158.6 114.5) (width 0.5) (layer "B.Cu") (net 8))
 (segment (start 155.1 113.5) (end 154.327 112.727) (width 0.5) (layer "B.Cu") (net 8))
 (segment (start 155.7 113.5) (end 156.7 114.5) (width 0.5) (layer "B.Cu") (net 8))
 (segment (start 142.4 98.5) (end 154.9 98.5) (width 0.5) (layer "B.Cu") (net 8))
 (segment (start 154.4 128.2) (end 154.4 114.2) (width 0.5) (layer "B.Cu") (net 8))
 (segment (start 154.327 107.723) (end 153.802 107.198) (width 0.5) (layer "B.Cu") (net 8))
 (segment (start 154.9 98.5) (end 158.6 98.5) (width 0.5) (layer "B.Cu") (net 8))
 (segment (start 158.6 130.5) (end 156.7 130.5) (width 0.5) (layer "B.Cu") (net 8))
 (segment (start 154.4 114.2) (end 155.1 113.5) (width 0.5) (layer "B.Cu") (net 8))
 (segment (start 154.327 112.727) (end 154.327 107.723) (width 0.5) (layer "B.Cu") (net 8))
 (segment (start 155.1 98.7) (end 154.9 98.5) (width 0.5) (layer "B.Cu") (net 8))
 (segment (start 156.7 130.5) (end 154.4 128.2) (width 0.5) (layer "B.Cu") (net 8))
 (segment (start 151.475 119.31) (end 154.19 119.31) (width 0.2) (layer "F.Cu") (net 4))
 (segment (start 154.19 119.31) (end 155.3 118.2) (width 0.2) (layer "F.Cu") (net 4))
 (segment (start 157.4 112.5) (end 158.65 112.5) (width 0.2) (layer "F.Cu") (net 4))
 (segment (start 155.3 114.6) (end 157.4 112.5) (width 0.2) (layer "F.Cu") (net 4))
 (via (at 155.3 118.2) (size 0.5) (drill 0.2) (layers "F.Cu" "B.Cu") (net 4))
 (via (at 155.3 114.6) (size 0.5) (drill 0.2) (layers "F.Cu" "B.Cu") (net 4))
 (segment (start 155.3 118.2) (end 155.223 118.123) (width 0.2) (layer "B.Cu") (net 4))
 (segment (start 155.223 114.677) (end 155.3 114.6) (width 0.2) (layer "B.Cu") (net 4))
 (segment (start 155.223 118.123) (end 155.223 114.677) (width 0.2) (layer "B.Cu") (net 4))
 (segment (start 155.8 115.5) (end 156.8 114.5) (width 0.2) (layer "F.Cu") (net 5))
 (segment (start 156.8 114.5) (end 158.65 114.5) (width 0.2) (layer "F.Cu") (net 5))
 (segment (start 151.475 118.04) (end 154.76 118.04) (width 0.2) (layer "F.Cu") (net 5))
 (segment (start 154.76 118.04) (end 155.7 117.1) (width 0.2) (layer "F.Cu") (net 5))
 (via (at 155.8 115.5) (size 0.5) (drill 0.2) (layers "F.Cu" "B.Cu") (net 5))
 (via (at 155.7 117.1) (size 0.5) (drill 0.2) (layers "F.Cu" "B.Cu") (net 5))
 (segment (start 155.7 117.1) (end 155.7 115.6) (width 0.2) (layer "B.Cu") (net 5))
 (segment (start 155.7 115.6) (end 155.8 115.5) (width 0.2) (layer "B.Cu") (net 5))
 (segment (start 151.745 116.5) (end 151.475 116.77) (width 0.2) (layer "F.Cu") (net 6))
 (segment (start 158.65 116.5) (end 151.745 116.5) (width 0.2) (layer "F.Cu") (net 6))
 (segment (start 156 112.4) (end 156 108.5) (width 0.2) (layer "F.Cu") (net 7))
 (segment (start 152.9 115.5) (end 154.7 113.7) (width 0.2) (layer "F.Cu") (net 7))
 (segment (start 154.7 113.7) (end 156 112.4) (width 0.2) (layer "F.Cu") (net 7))
 (segment (start 151.475 115.5) (end 152.9 115.5) (width 0.2) (layer "F.Cu") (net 7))
 (via (at 156 108.5) (size 0.5) (drill 0.2) (layers "F.Cu" "B.Cu") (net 7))
 (segment (start 156 108.5) (end 158.6 108.5) (width 0.2) (layer "B.Cu") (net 7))
 (segment (start 148.8 110.6) (end 148.8 94.5) (width 0.2) (layer "F.Cu") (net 12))
 (segment (start 156.5 95) (end 157 94.5) (width 0.2) (layer "F.Cu") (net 12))
 (segment (start 148.8 94.5) (end 154.4235 94.5) (width 0.2) (layer "F.Cu") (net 12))
 (segment (start 142.35 94.5) (end 148.8 94.5) (width 0.2) (layer "F.Cu") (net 12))
 (segment (start 151.385 111.6) (end 149.8 111.6) (width 0.2) (layer "F.Cu") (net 12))
 (segment (start 157 94.5) (end 158.65 94.5) (width 0.2) (layer "F.Cu") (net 12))
 (segment (start 154.4235 94.5) (end 154.9 94.9765) (width 0.2) (layer "F.Cu") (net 12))
 (segment (start 149.8 111.6) (end 148.8 110.6) (width 0.2) (layer "F.Cu") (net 12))
 (segment (start 151.475 111.69) (end 151.385 111.6) (width 0.2) (layer "F.Cu") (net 12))
 (via (at 154.9 94.9765) (size 0.5) (drill 0.2) (layers "F.Cu" "B.Cu") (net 12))
 (via (at 156.5 95) (size 0.5) (drill 0.2) (layers "F.Cu" "B.Cu") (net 12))
 (segment (start 154.9 94.9765) (end 156.4765 94.9765) (width 0.2) (layer "B.Cu") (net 12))
 (segment (start 156.4765 94.9765) (end 156.5 95) (width 0.2) (layer "B.Cu") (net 12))
 (segment (start 148.2 111.4) (end 148.3 111.3) (width 0.2) (layer "F.Cu") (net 13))
 (segment (start 145.2 96.5) (end 142.35 96.5) (width 0.2) (layer "F.Cu") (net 13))
 (segment (start 148.3 111.3) (end 148.3 96.5) (width 0.2) (layer "F.Cu") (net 13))
 (segment (start 146.525 111.69) (end 147.91 111.69) (width 0.2) (layer "F.Cu") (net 13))
 (segment (start 158.65 96.5) (end 156.4265 96.5) (width 0.2) (layer "F.Cu") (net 13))
 (segment (start 147.91 111.69) (end 148.2 111.4) (width 0.2) (layer "F.Cu") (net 13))
 (via (at 148.3 96.5) (size 0.5) (drill 0.2) (layers "F.Cu" "B.Cu") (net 13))
 (via (at 156.4265 96.5) (size 0.5) (drill 0.2) (layers "F.Cu" "B.Cu") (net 13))
 (via (at 145.2 96.5) (size 0.5) (drill 0.2) (layers "F.Cu" "B.Cu") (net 13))
 (segment (start 156.4265 96.5) (end 154.8 96.5) (width 0.2) (layer "B.Cu") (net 13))
 (segment (start 148.3 96.5) (end 154.8 96.5) (width 0.2) (layer "B.Cu") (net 13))
 (segment (start 148.3 96.5) (end 145.2 96.5) (width 0.2) (layer "B.Cu") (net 13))
 (segment (start 156.673 126.016159) (end 156.673 127.673) (width 0.2) (layer "F.Cu") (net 18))
 (segment (start 148.027 117.370159) (end 156.673 126.016159) (width 0.2) (layer "F.Cu") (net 18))
 (segment (start 146.763159 115.5) (end 148.027 116.763841) (width 0.2) (layer "F.Cu") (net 18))
 (segment (start 157.5 128.5) (end 158.65 128.5) (width 0.2) (layer "F.Cu") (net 18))
 (segment (start 156.673 127.673) (end 157.5 128.5) (width 0.2) (layer "F.Cu") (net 18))
 (segment (start 146.525 115.5) (end 146.763159 115.5) (width 0.2) (layer "F.Cu") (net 18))
 (segment (start 148.027 116.763841) (end 148.027 117.370159) (width 0.2) (layer "F.Cu") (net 18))
 (segment (start 147.27 116.77) (end 147.7 117.2) (width 0.2) (layer "F.Cu") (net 19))
 (segment (start 147.7 117.505607) (end 156.3 126.105607) (width 0.2) (layer "F.Cu") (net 19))
 (segment (start 156.3 126.105607) (end 156.3 129.8) (width 0.2) (layer "F.Cu") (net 19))
 (segment (start 146.525 116.77) (end 147.27 116.77) (width 0.2) (layer "F.Cu") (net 19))
 (segment (start 156.3 129.8) (end 157 130.5) (width 0.2) (layer "F.Cu") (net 19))
 (segment (start 147.7 117.2) (end 147.7 117.505607) (width 0.2) (layer "F.Cu") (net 19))
 (segment (start 157 130.5) (end 158.65 130.5) (width 0.2) (layer "F.Cu") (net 19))
 (segment (start 155.8 131.2) (end 155.8 126.068055) (width 0.2) (layer "F.Cu") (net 20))
 (segment (start 147.771945 118.04) (end 146.525 118.04) (width 0.2) (layer "F.Cu") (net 20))
 (segment (start 157.1 132.5) (end 155.8 131.2) (width 0.2) (layer "F.Cu") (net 20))
 (segment (start 158.65 132.5) (end 157.1 132.5) (width 0.2) (layer "F.Cu") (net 20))
 (segment (start 155.8 126.068055) (end 147.771945 118.04) (width 0.2) (layer "F.Cu") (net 20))
 (segment (start 155.1 125.830503) (end 148.569497 119.3) (width 0.2) (layer "F.Cu") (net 21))
 (segment (start 146.535 119.3) (end 146.525 119.31) (width 0.2) (layer "F.Cu") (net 21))
 (segment (start 155.1 126.3) (end 155.1 125.830503) (width 0.2) (layer "F.Cu") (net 21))
 (segment (start 147.9 119.3) (end 146.535 119.3) (width 0.2) (layer "F.Cu") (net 21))
 (segment (start 148.569497 119.3) (end 147.9 119.3) (width 0.2) (layer "F.Cu") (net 21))
 (via (at 155.1 126.3) (size 0.5) (drill 0.2) (layers "F.Cu" "B.Cu") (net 21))
 (segment (start 158.6 124.5) (end 156.9 124.5) (width 0.2) (layer "B.Cu") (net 21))
 (segment (start 156.9 124.5) (end 155.1 126.3) (width 0.2) (layer "B.Cu") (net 21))
 (segment (start 158.65 96.5) (end 157.4 96.5) (width 0.2) (layer "B.Cu") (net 16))
 (segment (start 145.1 95.9) (end 144.5 96.5) (width 0.2) (layer "B.Cu") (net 16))
 (segment (start 157.4 96.5) (end 156.8 95.9) (width 0.2) (layer "B.Cu") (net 16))
 (segment (start 156.8 95.9) (end 145.1 95.9) (width 0.2) (layer "B.Cu") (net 16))
 (segment (start 144.5 96.5) (end 142.6 96.5) (width 0.2) (layer "B.Cu") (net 16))
 (segment (start 143.527 114.877) (end 145.223 114.877) (width 0.2) (layer "F.Cu") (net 11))
 (segment (start 145.223 114.877) (end 145.87 114.23) (width 0.2) (layer "F.Cu") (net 11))
 (segment (start 142.9 114.25) (end 143.527 114.877) (width 0.2) (layer "F.Cu") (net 11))
 (segment (start 142.9 114.25) (end 142.9 112.9) (width 0.2) (layer "F.Cu") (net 11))
 (segment (start 145.87 114.23) (end 146.048 114.23) (width 0.2) (layer "F.Cu") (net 11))
 (segment (start 144.4 112.9) (end 144.4 114.25) (width 0.2) (layer "F.Cu") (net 10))
 (segment (start 144.46 112.96) (end 144.4 112.9) (width 0.2) (layer "F.Cu") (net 10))
 (segment (start 146.525 112.96) (end 144.46 112.96) (width 0.2) (layer "F.Cu") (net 10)))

